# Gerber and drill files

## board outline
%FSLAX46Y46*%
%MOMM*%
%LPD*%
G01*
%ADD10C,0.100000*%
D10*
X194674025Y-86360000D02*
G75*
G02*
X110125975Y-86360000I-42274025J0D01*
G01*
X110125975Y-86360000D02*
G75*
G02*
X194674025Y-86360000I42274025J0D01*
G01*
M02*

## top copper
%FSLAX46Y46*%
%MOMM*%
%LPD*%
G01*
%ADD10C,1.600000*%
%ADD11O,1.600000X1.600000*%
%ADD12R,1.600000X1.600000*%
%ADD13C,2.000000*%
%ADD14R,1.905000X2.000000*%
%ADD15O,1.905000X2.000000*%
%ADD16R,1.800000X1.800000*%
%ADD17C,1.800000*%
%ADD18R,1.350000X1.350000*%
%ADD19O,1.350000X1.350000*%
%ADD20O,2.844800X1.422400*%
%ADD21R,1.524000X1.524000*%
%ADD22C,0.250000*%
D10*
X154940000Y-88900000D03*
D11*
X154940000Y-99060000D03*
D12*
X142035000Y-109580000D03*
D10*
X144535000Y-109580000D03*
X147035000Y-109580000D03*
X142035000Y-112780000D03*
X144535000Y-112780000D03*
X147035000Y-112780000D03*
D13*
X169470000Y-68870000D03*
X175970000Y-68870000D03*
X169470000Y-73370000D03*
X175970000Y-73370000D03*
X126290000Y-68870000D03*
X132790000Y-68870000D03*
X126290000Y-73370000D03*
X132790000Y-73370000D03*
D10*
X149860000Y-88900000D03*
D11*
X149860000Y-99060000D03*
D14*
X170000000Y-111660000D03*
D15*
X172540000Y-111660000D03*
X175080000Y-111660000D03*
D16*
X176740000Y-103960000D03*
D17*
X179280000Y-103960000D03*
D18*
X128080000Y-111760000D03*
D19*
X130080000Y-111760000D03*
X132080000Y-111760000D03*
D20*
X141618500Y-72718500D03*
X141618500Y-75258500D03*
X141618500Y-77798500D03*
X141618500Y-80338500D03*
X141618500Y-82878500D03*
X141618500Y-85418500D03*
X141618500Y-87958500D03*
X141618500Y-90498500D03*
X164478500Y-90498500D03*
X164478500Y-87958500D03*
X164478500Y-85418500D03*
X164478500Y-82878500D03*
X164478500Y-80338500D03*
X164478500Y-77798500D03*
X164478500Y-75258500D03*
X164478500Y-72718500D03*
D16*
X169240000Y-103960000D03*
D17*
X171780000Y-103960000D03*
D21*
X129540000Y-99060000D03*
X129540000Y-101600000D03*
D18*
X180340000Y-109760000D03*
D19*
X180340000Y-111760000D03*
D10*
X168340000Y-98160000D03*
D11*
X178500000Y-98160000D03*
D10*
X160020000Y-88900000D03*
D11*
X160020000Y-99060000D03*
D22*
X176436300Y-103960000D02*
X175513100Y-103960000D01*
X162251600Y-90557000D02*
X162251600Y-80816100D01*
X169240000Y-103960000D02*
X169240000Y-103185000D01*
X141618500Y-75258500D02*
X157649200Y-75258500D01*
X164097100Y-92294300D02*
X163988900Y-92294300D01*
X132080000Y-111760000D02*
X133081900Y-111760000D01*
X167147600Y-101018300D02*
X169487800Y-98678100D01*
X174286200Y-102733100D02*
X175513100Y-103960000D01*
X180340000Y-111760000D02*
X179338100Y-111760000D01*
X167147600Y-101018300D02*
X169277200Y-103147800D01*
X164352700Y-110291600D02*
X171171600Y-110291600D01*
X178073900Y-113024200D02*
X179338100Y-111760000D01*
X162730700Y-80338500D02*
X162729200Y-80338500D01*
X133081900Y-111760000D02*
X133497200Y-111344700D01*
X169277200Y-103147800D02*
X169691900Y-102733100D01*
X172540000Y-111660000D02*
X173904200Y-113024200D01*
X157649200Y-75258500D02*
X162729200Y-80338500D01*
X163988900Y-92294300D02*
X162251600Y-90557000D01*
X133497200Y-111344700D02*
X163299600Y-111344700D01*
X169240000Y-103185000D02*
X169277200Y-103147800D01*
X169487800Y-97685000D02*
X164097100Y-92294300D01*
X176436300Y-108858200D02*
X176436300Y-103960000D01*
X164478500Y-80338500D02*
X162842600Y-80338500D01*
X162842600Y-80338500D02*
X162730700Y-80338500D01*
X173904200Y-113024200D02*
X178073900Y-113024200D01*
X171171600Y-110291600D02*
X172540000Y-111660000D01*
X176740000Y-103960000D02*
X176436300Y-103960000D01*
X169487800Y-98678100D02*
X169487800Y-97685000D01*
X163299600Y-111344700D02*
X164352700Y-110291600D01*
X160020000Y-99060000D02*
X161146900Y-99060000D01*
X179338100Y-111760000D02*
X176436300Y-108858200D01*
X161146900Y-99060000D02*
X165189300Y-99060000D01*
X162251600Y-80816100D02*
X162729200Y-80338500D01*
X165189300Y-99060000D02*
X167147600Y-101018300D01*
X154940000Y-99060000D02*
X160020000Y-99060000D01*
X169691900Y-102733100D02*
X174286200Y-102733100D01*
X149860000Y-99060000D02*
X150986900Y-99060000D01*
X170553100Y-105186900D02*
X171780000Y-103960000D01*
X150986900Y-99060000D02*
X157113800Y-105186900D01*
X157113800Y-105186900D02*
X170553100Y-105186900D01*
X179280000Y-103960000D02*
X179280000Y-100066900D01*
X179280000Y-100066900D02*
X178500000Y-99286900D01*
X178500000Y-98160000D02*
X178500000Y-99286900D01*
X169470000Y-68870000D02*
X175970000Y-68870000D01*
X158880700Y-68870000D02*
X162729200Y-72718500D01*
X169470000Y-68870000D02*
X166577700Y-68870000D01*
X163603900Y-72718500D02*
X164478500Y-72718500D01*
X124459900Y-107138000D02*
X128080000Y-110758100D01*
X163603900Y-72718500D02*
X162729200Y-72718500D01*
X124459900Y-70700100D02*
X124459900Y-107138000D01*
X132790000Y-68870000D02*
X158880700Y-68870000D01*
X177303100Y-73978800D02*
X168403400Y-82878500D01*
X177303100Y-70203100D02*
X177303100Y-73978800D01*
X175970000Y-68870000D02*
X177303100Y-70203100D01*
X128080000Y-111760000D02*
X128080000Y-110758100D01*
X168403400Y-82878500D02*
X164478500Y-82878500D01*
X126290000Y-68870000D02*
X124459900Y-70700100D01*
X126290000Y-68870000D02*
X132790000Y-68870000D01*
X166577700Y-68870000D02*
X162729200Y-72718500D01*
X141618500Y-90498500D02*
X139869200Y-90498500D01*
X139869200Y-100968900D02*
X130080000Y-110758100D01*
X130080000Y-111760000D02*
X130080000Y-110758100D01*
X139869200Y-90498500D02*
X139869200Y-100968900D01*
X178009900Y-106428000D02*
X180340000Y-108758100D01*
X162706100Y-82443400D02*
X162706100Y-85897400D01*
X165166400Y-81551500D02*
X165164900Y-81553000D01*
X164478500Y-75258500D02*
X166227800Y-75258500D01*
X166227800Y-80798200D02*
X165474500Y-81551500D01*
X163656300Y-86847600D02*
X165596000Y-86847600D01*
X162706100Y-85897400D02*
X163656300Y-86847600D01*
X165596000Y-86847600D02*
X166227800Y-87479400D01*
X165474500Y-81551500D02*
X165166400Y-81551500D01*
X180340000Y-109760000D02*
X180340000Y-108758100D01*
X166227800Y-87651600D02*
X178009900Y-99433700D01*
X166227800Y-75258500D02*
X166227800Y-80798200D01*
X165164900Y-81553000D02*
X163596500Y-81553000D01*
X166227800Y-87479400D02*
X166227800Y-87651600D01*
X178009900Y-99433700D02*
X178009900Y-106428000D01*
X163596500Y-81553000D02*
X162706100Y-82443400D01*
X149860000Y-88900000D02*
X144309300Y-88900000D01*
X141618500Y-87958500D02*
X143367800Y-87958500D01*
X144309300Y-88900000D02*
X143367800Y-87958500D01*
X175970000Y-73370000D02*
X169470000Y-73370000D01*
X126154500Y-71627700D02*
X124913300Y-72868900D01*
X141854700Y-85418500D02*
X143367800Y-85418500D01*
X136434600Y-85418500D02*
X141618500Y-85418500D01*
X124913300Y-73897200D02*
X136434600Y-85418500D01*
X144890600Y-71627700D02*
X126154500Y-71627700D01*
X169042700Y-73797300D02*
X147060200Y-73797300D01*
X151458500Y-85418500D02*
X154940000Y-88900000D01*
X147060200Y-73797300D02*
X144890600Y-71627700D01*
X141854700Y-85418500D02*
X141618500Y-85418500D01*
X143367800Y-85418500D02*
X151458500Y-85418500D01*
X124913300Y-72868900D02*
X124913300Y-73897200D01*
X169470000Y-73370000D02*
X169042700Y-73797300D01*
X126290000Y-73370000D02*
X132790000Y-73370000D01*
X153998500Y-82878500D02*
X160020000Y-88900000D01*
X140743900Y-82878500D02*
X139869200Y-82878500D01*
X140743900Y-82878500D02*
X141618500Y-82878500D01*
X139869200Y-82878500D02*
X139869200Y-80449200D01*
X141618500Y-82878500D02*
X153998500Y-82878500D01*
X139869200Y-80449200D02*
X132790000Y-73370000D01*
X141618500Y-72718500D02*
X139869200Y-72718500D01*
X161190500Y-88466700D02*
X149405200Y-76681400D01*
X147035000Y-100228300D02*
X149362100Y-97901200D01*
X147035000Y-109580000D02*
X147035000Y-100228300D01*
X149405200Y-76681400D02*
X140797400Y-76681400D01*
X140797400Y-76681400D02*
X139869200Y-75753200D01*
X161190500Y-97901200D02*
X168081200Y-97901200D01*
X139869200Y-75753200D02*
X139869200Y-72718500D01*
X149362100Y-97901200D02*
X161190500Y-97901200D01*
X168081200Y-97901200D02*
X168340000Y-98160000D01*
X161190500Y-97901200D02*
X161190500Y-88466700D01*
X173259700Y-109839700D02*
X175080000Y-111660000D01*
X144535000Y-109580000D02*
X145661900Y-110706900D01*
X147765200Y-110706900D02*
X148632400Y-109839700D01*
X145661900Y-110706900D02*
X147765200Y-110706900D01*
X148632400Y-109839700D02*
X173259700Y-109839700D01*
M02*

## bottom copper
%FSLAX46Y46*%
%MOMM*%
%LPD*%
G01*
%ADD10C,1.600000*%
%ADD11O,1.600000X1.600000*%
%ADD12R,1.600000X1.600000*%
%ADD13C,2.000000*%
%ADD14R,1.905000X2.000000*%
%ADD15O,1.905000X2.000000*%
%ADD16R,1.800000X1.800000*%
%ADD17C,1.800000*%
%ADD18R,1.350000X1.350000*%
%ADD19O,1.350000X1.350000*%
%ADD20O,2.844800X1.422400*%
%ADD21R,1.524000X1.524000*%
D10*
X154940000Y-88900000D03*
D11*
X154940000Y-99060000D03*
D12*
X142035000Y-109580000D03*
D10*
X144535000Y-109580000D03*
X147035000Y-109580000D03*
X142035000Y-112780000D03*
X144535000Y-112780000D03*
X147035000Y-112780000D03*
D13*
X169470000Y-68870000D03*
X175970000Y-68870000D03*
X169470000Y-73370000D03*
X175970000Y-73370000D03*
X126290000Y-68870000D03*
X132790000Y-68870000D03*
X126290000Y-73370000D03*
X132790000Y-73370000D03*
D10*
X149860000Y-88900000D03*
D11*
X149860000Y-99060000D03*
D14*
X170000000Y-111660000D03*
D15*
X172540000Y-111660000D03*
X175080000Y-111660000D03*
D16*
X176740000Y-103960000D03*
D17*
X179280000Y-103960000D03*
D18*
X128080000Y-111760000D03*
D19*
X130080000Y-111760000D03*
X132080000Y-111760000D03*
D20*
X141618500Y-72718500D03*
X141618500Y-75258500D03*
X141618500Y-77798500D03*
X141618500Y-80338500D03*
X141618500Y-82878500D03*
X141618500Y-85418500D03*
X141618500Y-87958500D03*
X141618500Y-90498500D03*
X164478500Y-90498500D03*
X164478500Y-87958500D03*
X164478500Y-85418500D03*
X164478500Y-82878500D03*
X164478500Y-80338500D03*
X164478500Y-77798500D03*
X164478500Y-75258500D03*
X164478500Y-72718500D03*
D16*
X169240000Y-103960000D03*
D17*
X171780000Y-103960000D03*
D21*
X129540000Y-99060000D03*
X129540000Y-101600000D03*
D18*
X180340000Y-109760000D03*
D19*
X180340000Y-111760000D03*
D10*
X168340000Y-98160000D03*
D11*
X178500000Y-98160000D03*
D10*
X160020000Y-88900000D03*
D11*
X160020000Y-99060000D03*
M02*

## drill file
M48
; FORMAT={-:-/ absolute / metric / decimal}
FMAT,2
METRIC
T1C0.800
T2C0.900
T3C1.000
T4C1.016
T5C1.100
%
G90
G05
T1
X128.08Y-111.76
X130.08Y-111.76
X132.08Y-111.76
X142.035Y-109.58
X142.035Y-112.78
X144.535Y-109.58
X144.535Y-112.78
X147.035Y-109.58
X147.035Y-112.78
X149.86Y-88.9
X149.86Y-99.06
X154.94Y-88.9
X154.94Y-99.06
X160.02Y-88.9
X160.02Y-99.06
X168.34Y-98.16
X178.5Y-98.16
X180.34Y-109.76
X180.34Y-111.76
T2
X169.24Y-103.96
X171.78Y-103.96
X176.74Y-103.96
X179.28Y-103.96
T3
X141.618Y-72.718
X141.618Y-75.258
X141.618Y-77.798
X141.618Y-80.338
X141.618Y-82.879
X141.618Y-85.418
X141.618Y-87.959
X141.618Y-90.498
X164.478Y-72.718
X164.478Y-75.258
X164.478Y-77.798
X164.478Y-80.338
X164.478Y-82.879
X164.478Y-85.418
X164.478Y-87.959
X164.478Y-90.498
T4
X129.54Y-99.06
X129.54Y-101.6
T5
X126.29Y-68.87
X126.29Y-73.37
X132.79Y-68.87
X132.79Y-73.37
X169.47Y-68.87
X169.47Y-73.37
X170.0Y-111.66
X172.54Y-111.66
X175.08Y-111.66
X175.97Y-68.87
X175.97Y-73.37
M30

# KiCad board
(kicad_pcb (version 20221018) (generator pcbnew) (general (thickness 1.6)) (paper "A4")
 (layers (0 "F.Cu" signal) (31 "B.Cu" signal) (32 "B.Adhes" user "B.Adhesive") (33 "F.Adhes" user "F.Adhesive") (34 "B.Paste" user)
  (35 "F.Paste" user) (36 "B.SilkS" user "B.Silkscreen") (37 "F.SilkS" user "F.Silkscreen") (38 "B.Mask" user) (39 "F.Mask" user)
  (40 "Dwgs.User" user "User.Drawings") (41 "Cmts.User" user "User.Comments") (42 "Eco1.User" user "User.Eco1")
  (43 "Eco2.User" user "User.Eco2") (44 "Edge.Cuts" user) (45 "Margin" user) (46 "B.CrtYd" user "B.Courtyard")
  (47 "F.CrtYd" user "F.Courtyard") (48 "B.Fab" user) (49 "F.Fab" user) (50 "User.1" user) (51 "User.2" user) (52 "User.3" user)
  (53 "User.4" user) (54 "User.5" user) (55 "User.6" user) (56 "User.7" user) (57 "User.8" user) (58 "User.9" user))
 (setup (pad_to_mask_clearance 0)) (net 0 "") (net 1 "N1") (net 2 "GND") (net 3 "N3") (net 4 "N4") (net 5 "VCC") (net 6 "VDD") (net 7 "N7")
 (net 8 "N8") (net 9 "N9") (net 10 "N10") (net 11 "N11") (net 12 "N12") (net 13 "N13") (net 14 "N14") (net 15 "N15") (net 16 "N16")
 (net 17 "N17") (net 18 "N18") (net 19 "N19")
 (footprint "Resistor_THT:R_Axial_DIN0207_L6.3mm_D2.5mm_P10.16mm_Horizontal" (layer "F.Cu") (at 154.94 88.9 -90)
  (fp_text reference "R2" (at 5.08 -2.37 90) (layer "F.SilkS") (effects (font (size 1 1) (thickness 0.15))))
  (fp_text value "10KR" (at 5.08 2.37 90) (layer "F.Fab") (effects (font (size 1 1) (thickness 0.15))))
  (pad "1" thru_hole circle (at 0 0 270) (size 1.6 1.6) (drill 0.8) (layers "*.Cu" "*.Mask") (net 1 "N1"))
  (pad "2" thru_hole oval (at 10.16 0 270) (size 1.6 1.6) (drill 0.8) (layers "*.Cu" "*.Mask") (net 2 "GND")))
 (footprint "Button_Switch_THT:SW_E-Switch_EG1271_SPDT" (layer "F.Cu") (at 142.035 109.58)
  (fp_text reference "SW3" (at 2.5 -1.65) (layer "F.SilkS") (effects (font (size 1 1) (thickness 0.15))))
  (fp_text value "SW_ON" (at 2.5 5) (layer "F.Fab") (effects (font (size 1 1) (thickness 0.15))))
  (pad "1" thru_hole rect (at 0 0) (size 1.6 1.6) (drill 0.8) (layers "*.Cu" "*.Mask") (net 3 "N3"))
  (pad "2" thru_hole circle (at 2.5 0) (size 1.6 1.6) (drill 0.8) (layers "*.Cu" "*.Mask") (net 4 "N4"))
  (pad "3" thru_hole circle (at 5 0) (size 1.6 1.6) (drill 0.8) (layers "*.Cu" "*.Mask") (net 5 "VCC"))
  (pad "4" thru_hole circle (at 0 3.2) (size 1.6 1.6) (drill 0.8) (layers "*.Cu" "*.Mask"))
  (pad "5" thru_hole circle (at 2.5 3.2) (size 1.6 1.6) (drill 0.8) (layers "*.Cu" "*.Mask"))
  (pad "6" thru_hole circle (at 5 3.2) (size 1.6 1.6) (drill 0.8) (layers "*.Cu" "*.Mask")))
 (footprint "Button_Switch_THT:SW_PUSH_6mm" (layer "F.Cu") (at 169.47 68.87)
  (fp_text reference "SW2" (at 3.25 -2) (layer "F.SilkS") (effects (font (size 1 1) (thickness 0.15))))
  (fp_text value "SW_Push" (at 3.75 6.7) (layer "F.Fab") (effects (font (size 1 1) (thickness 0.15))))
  (pad "1" thru_hole circle (at 0 0 90) (size 2 2) (drill 1.1) (layers "*.Cu" "*.Mask") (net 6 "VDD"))
  (pad "1" thru_hole circle (at 6.5 0 90) (size 2 2) (drill 1.1) (layers "*.Cu" "*.Mask") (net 6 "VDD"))
  (pad "2" thru_hole circle (at 0 4.5 90) (size 2 2) (drill 1.1) (layers "*.Cu" "*.Mask") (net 1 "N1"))
  (pad "2" thru_hole circle (at 6.5 4.5 90) (size 2 2) (drill 1.1) (layers "*.Cu" "*.Mask") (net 1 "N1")))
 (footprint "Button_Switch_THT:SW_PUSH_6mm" (layer "F.Cu") (at 126.29 68.87)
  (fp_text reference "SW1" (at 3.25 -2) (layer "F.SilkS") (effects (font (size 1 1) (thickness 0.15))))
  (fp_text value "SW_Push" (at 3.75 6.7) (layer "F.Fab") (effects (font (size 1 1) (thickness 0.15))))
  (pad "1" thru_hole circle (at 0 0 90) (size 2 2) (drill 1.1) (layers "*.Cu" "*.Mask") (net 6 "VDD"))
  (pad "1" thru_hole circle (at 6.5 0 90) (size 2 2) (drill 1.1) (layers "*.Cu" "*.Mask") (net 6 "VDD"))
  (pad "2" thru_hole circle (at 0 4.5 90) (size 2 2) (drill 1.1) (layers "*.Cu" "*.Mask") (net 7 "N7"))
  (pad "2" thru_hole circle (at 6.5 4.5 90) (size 2 2) (drill 1.1) (layers "*.Cu" "*.Mask") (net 7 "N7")))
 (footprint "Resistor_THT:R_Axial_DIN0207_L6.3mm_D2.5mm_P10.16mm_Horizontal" (layer "F.Cu") (at 149.86 88.9 -90)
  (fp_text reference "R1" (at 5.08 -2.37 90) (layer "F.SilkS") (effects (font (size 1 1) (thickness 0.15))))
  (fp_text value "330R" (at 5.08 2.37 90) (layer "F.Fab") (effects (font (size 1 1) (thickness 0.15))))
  (pad "1" thru_hole circle (at 0 0 270) (size 1.6 1.6) (drill 0.8) (layers "*.Cu" "*.Mask") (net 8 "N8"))
  (pad "2" thru_hole oval (at 10.16 0 270) (size 1.6 1.6) (drill 0.8) (layers "*.Cu" "*.Mask") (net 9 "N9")))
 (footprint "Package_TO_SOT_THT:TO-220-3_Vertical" (layer "F.Cu") (at 170 111.66)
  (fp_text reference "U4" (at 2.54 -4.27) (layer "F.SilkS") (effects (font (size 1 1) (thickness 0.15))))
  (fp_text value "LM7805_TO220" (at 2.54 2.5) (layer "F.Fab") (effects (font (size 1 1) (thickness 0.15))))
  (pad "1" thru_hole rect (at 0 0) (size 1.905 2) (drill 1.1) (layers "*.Cu" "*.Mask") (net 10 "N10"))
  (pad "2" thru_hole oval (at 2.54 0) (size 1.905 2) (drill 1.1) (layers "*.Cu" "*.Mask") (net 2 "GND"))
  (pad "3" thru_hole oval (at 5.08 0) (size 1.905 2) (drill 1.1) (layers "*.Cu" "*.Mask") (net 4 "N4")))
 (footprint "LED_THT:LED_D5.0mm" (layer "F.Cu") (at 176.74 103.96)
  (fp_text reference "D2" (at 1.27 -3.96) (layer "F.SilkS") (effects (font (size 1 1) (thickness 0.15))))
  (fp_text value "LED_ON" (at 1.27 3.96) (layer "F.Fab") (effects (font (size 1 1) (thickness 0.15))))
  (pad "1" thru_hole rect (at 0 0) (size 1.8 1.8) (drill 0.9) (layers "*.Cu" "*.Mask") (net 2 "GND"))
  (pad "2" thru_hole circle (at 2.54 0) (size 1.8 1.8) (drill 0.9) (layers "*.Cu" "*.Mask") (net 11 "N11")))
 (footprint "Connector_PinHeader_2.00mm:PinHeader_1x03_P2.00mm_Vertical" (layer "F.Cu") (at 128.08 111.76 90)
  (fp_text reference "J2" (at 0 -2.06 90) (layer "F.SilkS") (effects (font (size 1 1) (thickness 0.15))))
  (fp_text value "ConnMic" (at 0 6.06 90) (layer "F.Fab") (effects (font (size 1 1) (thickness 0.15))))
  (pad "1" thru_hole rect (at 0 0 90) (size 1.35 1.35) (drill 0.8) (layers "*.Cu" "*.Mask") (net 6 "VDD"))
  (pad "2" thru_hole oval (at 0 2 90) (size 1.35 1.35) (drill 0.8) (layers "*.Cu" "*.Mask") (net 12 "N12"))
  (pad "3" thru_hole oval (at 0 4 90) (size 1.35 1.35) (drill 0.8) (layers "*.Cu" "*.Mask") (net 2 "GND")))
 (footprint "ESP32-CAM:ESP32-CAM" (layer "F.Cu") (at 153.0485 82.8785)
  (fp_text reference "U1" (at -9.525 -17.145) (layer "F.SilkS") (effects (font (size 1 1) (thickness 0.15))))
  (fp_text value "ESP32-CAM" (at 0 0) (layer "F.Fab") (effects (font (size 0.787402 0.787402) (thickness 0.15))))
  (pad "P$1" thru_hole oval (at -11.43 -10.16) (size 2.8448 1.4224) (drill 1) (layers "*.Cu" "*.Mask") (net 5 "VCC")
   (solder_mask_margin 0.102))
  (pad "P$2" thru_hole oval (at -11.43 -7.62) (size 2.8448 1.4224) (drill 1) (layers "*.Cu" "*.Mask") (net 2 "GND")
   (solder_mask_margin 0.102))
  (pad "P$3" thru_hole oval (at -11.43 -5.08) (size 2.8448 1.4224) (drill 1) (layers "*.Cu" "*.Mask") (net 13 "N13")
   (solder_mask_margin 0.102))
  (pad "P$4" thru_hole oval (at -11.43 -2.54) (size 2.8448 1.4224) (drill 1) (layers "*.Cu" "*.Mask") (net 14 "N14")
   (solder_mask_margin 0.102))
  (pad "P$5" thru_hole oval (at -11.43 0) (size 2.8448 1.4224) (drill 1) (layers "*.Cu" "*.Mask") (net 7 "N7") (solder_mask_margin 0.102))
  (pad "P$6" thru_hole oval (at -11.43 2.54) (size 2.8448 1.4224) (drill 1) (layers "*.Cu" "*.Mask") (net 1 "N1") (solder_mask_margin 0.102))
  (pad "P$7" thru_hole oval (at -11.43 5.08) (size 2.8448 1.4224) (drill 1) (layers "*.Cu" "*.Mask") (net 8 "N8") (solder_mask_margin 0.102))
  (pad "P$8" thru_hole oval (at -11.43 7.62) (size 2.8448 1.4224) (drill 1) (layers "*.Cu" "*.Mask") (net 12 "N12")
   (solder_mask_margin 0.102))
  (pad "P$9" thru_hole oval (at 11.43 7.62) (size 2.8448 1.4224) (drill 1) (layers "*.Cu" "*.Mask") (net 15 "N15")
   (solder_mask_margin 0.102))
  (pad "P$10" thru_hole oval (at 11.43 5.08) (size 2.8448 1.4224) (drill 1) (layers "*.Cu" "*.Mask") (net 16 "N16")
   (solder_mask_margin 0.102))
  (pad "P$11" thru_hole oval (at 11.43 2.54) (size 2.8448 1.4224) (drill 1) (layers "*.Cu" "*.Mask") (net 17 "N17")
   (solder_mask_margin 0.102))
  (pad "P$12" thru_hole oval (at 11.43 0) (size 2.8448 1.4224) (drill 1) (layers "*.Cu" "*.Mask") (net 6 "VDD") (solder_mask_margin 0.102))
  (pad "P$13" thru_hole oval (at 11.43 -2.54) (size 2.8448 1.4224) (drill 1) (layers "*.Cu" "*.Mask") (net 2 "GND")
   (solder_mask_margin 0.102))
  (pad "P$14" thru_hole oval (at 11.43 -5.08) (size 2.8448 1.4224) (drill 1) (layers "*.Cu" "*.Mask") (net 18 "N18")
   (solder_mask_margin 0.102))
  (pad "P$15" thru_hole oval (at 11.43 -7.62) (size 2.8448 1.4224) (drill 1) (layers "*.Cu" "*.Mask") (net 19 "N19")
   (solder_mask_margin 0.102))
  (pad "P$16" thru_hole oval (at 11.43 -10.16) (size 2.8448 1.4224) (drill 1) (layers "*.Cu" "*.Mask") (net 6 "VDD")
   (solder_mask_margin 0.102)))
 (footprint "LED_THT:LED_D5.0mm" (layer "F.Cu") (at 169.24 103.96)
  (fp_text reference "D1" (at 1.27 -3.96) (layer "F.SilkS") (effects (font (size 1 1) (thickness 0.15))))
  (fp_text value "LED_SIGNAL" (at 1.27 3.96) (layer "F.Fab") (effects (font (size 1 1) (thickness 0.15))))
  (pad "1" thru_hole rect (at 0 0) (size 1.8 1.8) (drill 0.9) (layers "*.Cu" "*.Mask") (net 2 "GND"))
  (pad "2" thru_hole circle (at 2.54 0) (size 1.8 1.8) (drill 0.9) (layers "*.Cu" "*.Mask") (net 9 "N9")))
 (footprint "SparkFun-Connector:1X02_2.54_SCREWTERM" (layer "F.Cu") (at 129.54 101.6 90)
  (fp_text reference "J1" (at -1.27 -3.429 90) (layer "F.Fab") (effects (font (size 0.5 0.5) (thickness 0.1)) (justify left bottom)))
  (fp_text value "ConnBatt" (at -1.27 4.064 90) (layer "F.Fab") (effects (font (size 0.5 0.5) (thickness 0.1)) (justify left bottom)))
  (pad "P1" thru_hole rect (at 2.54 0 90) (size 1.524 1.524) (drill 1.016) (layers "*.Cu" "*.Mask") (solder_mask_margin 0.1016)
   (thermal_bridge_angle 45))
  (pad "P2" thru_hole rect (at 0 0 90) (size 1.524 1.524) (drill 1.016) (layers "*.Cu" "*.Mask") (solder_mask_margin 0.1016)
   (thermal_bridge_angle 45)))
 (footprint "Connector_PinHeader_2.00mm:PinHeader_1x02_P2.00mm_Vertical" (layer "F.Cu") (at 180.34 109.76)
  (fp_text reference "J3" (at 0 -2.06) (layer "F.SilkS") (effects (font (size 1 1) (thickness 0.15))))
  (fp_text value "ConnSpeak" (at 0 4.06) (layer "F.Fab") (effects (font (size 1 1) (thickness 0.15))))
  (pad "1" thru_hole rect (at 0 0) (size 1.35 1.35) (drill 0.8) (layers "*.Cu" "*.Mask") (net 19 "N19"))
  (pad "2" thru_hole oval (at 0 2) (size 1.35 1.35) (drill 0.8) (layers "*.Cu" "*.Mask") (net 2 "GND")))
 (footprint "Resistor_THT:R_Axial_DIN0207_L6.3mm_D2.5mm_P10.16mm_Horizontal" (layer "F.Cu") (at 168.34 98.16)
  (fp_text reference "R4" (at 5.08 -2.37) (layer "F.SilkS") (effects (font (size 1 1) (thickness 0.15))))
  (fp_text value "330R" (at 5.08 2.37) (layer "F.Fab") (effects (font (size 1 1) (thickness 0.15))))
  (pad "1" thru_hole circle (at 0 0) (size 1.6 1.6) (drill 0.8) (layers "*.Cu" "*.Mask") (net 5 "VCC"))
  (pad "2" thru_hole oval (at 10.16 0) (size 1.6 1.6) (drill 0.8) (layers "*.Cu" "*.Mask") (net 11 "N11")))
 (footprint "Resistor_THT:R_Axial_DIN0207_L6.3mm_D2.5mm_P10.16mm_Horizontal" (layer "F.Cu") (at 160.02 88.9 -90)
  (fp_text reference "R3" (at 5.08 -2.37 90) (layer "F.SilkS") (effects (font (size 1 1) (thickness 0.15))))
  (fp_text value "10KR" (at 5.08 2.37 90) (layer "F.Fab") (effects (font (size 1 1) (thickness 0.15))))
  (pad "1" thru_hole circle (at 0 0 270) (size 1.6 1.6) (drill 0.8) (layers "*.Cu" "*.Mask") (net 7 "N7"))
  (pad "2" thru_hole oval (at 10.16 0 270) (size 1.6 1.6) (drill 0.8) (layers "*.Cu" "*.Mask") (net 2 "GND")))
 (gr_circle (center 152.4 86.36) (end 187.96 63.5) (stroke (width 0.1) (type default)) (fill none) (layer "Edge.Cuts"))
 (segment (start 176.4363 103.96) (end 175.5131 103.96) (width 0.25) (layer "F.Cu") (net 2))
 (segment (start 162.2516 90.557) (end 162.2516 80.8161) (width 0.25) (layer "F.Cu") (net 2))
 (segment (start 169.24 103.96) (end 169.24 103.185) (width 0.25) (layer "F.Cu") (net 2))
 (segment (start 141.6185 75.2585) (end 157.6492 75.2585) (width 0.25) (layer "F.Cu") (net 2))
 (segment (start 164.0971 92.2943) (end 163.9889 92.2943) (width 0.25) (layer "F.Cu") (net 2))
 (segment (start 132.08 111.76) (end 133.0819 111.76) (width 0.25) (layer "F.Cu") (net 2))
 (segment (start 167.1476 101.0183) (end 169.4878 98.6781) (width 0.25) (layer "F.Cu") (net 2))
 (segment (start 174.2862 102.7331) (end 175.5131 103.96) (width 0.25) (layer "F.Cu") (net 2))
 (segment (start 180.34 111.76) (end 179.3381 111.76) (width 0.25) (layer "F.Cu") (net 2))
 (segment (start 167.1476 101.0183) (end 169.2772 103.1478) (width 0.25) (layer "F.Cu") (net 2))
 (segment (start 164.3527 110.2916) (end 171.1716 110.2916) (width 0.25) (layer "F.Cu") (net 2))
 (segment (start 178.0739 113.0242) (end 179.3381 111.76) (width 0.25) (layer "F.Cu") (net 2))
 (segment (start 162.7307 80.3385) (end 162.7292 80.3385) (width 0.25) (layer "F.Cu") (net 2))
 (segment (start 133.0819 111.76) (end 133.4972 111.3447) (width 0.25) (layer "F.Cu") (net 2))
 (segment (start 169.2772 103.1478) (end 169.6919 102.7331) (width 0.25) (layer "F.Cu") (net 2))
 (segment (start 172.54 111.66) (end 173.9042 113.0242) (width 0.25) (layer "F.Cu") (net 2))
 (segment (start 157.6492 75.2585) (end 162.7292 80.3385) (width 0.25) (layer "F.Cu") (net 2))
 (segment (start 163.9889 92.2943) (end 162.2516 90.557) (width 0.25) (layer "F.Cu") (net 2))
 (segment (start 133.4972 111.3447) (end 163.2996 111.3447) (width 0.25) (layer "F.Cu") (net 2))
 (segment (start 169.24 103.185) (end 169.2772 103.1478) (width 0.25) (layer "F.Cu") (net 2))
 (segment (start 169.4878 97.685) (end 164.0971 92.2943) (width 0.25) (layer "F.Cu") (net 2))
 (segment (start 176.4363 108.8582) (end 176.4363 103.96) (width 0.25) (layer "F.Cu") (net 2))
 (segment (start 164.4785 80.3385) (end 162.8426 80.3385) (width 0.25) (layer "F.Cu") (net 2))
 (segment (start 162.8426 80.3385) (end 162.7307 80.3385) (width 0.25) (layer "F.Cu") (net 2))
 (segment (start 173.9042 113.0242) (end 178.0739 113.0242) (width 0.25) (layer "F.Cu") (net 2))
 (segment (start 171.1716 110.2916) (end 172.54 111.66) (width 0.25) (layer "F.Cu") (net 2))
 (segment (start 176.74 103.96) (end 176.4363 103.96) (width 0.25) (layer "F.Cu") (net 2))
 (segment (start 169.4878 98.6781) (end 169.4878 97.685) (width 0.25) (layer "F.Cu") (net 2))
 (segment (start 163.2996 111.3447) (end 164.3527 110.2916) (width 0.25) (layer "F.Cu") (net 2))
 (segment (start 160.02 99.06) (end 161.1469 99.06) (width 0.25) (layer "F.Cu") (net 2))
 (segment (start 179.3381 111.76) (end 176.4363 108.8582) (width 0.25) (layer "F.Cu") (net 2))
 (segment (start 161.1469 99.06) (end 165.1893 99.06) (width 0.25) (layer "F.Cu") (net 2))
 (segment (start 162.2516 80.8161) (end 162.7292 80.3385) (width 0.25) (layer "F.Cu") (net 2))
 (segment (start 165.1893 99.06) (end 167.1476 101.0183) (width 0.25) (layer "F.Cu") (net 2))
 (segment (start 154.94 99.06) (end 160.02 99.06) (width 0.25) (layer "F.Cu") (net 2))
 (segment (start 169.6919 102.7331) (end 174.2862 102.7331) (width 0.25) (layer "F.Cu") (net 2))
 (segment (start 149.86 99.06) (end 150.9869 99.06) (width 0.25) (layer "F.Cu") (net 9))
 (segment (start 170.5531 105.1869) (end 171.78 103.96) (width 0.25) (layer "F.Cu") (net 9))
 (segment (start 150.9869 99.06) (end 157.1138 105.1869) (width 0.25) (layer "F.Cu") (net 9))
 (segment (start 157.1138 105.1869) (end 170.5531 105.1869) (width 0.25) (layer "F.Cu") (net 9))
 (segment (start 179.28 103.96) (end 179.28 100.0669) (width 0.25) (layer "F.Cu") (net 11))
 (segment (start 179.28 100.0669) (end 178.5 99.2869) (width 0.25) (layer "F.Cu") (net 11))
 (segment (start 178.5 98.16) (end 178.5 99.2869) (width 0.25) (layer "F.Cu") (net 11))
 (segment (start 169.47 68.87) (end 175.97 68.87) (width 0.25) (layer "F.Cu") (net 6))
 (segment (start 158.8807 68.87) (end 162.7292 72.7185) (width 0.25) (layer "F.Cu") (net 6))
 (segment (start 169.47 68.87) (end 166.5777 68.87) (width 0.25) (layer "F.Cu") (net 6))
 (segment (start 163.6039 72.7185) (end 164.4785 72.7185) (width 0.25) (layer "F.Cu") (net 6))
 (segment (start 124.4599 107.138) (end 128.08 110.7581) (width 0.25) (layer "F.Cu") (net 6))
 (segment (start 163.6039 72.7185) (end 162.7292 72.7185) (width 0.25) (layer "F.Cu") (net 6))
 (segment (start 124.4599 70.7001) (end 124.4599 107.138) (width 0.25) (layer "F.Cu") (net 6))
 (segment (start 132.79 68.87) (end 158.8807 68.87) (width 0.25) (layer "F.Cu") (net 6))
 (segment (start 177.3031 73.9788) (end 168.4034 82.8785) (width 0.25) (layer "F.Cu") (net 6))
 (segment (start 177.3031 70.2031) (end 177.3031 73.9788) (width 0.25) (layer "F.Cu") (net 6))
 (segment (start 175.97 68.87) (end 177.3031 70.2031) (width 0.25) (layer "F.Cu") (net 6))
 (segment (start 128.08 111.76) (end 128.08 110.7581) (width 0.25) (layer "F.Cu") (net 6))
 (segment (start 168.4034 82.8785) (end 164.4785 82.8785) (width 0.25) (layer "F.Cu") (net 6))
 (segment (start 126.29 68.87) (end 124.4599 70.7001) (width 0.25) (layer "F.Cu") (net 6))
 (segment (start 126.29 68.87) (end 132.79 68.87) (width 0.25) (layer "F.Cu") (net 6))
 (segment (start 166.5777 68.87) (end 162.7292 72.7185) (width 0.25) (layer "F.Cu") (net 6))
 (segment (start 141.6185 90.4985) (end 139.8692 90.4985) (width 0.25) (layer "F.Cu") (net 12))
 (segment (start 139.8692 100.9689) (end 130.08 110.7581) (width 0.25) (layer "F.Cu") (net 12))
 (segment (start 130.08 111.76) (end 130.08 110.7581) (width 0.25) (layer "F.Cu") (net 12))
 (segment (start 139.8692 90.4985) (end 139.8692 100.9689) (width 0.25) (layer "F.Cu") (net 12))
 (segment (start 178.0099 106.428) (end 180.34 108.7581) (width 0.25) (layer "F.Cu") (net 19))
 (segment (start 162.7061 82.4434) (end 162.7061 85.8974) (width 0.25) (layer "F.Cu") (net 19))
 (segment (start 165.1664 81.5515) (end 165.1649 81.553) (width 0.25) (layer "F.Cu") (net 19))
 (segment (start 164.4785 75.2585) (end 166.2278 75.2585) (width 0.25) (layer "F.Cu") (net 19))
 (segment (start 166.2278 80.7982) (end 165.4745 81.5515) (width 0.25) (layer "F.Cu") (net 19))
 (segment (start 163.6563 86.8476) (end 165.596 86.8476) (width 0.25) (layer "F.Cu") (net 19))
 (segment (start 162.7061 85.8974) (end 163.6563 86.8476) (width 0.25) (layer "F.Cu") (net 19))
 (segment (start 165.596 86.8476) (end 166.2278 87.4794) (width 0.25) (layer "F.Cu") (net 19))
 (segment (start 165.4745 81.5515) (end 165.1664 81.5515) (width 0.25) (layer "F.Cu") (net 19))
 (segment (start 180.34 109.76) (end 180.34 108.7581) (width 0.25) (layer "F.Cu") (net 19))
 (segment (start 166.2278 87.6516) (end 178.0099 99.4337) (width 0.25) (layer "F.Cu") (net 19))
 (segment (start 166.2278 75.2585) (end 166.2278 80.7982) (width 0.25) (layer "F.Cu") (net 19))
 (segment (start 165.1649 81.553) (end 163.5965 81.553) (width 0.25) (layer "F.Cu") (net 19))
 (segment (start 166.2278 87.4794) (end 166.2278 87.6516) (width 0.25) (layer "F.Cu") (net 19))
 (segment (start 178.0099 99.4337) (end 178.0099 106.428) (width 0.25) (layer "F.Cu") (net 19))
 (segment (start 163.5965 81.553) (end 162.7061 82.4434) (width 0.25) (layer "F.Cu") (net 19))
 (segment (start 149.86 88.9) (end 144.3093 88.9) (width 0.25) (layer "F.Cu") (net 8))
 (segment (start 141.6185 87.9585) (end 143.3678 87.9585) (width 0.25) (layer "F.Cu") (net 8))
 (segment (start 144.3093 88.9) (end 143.3678 87.9585) (width 0.25) (layer "F.Cu") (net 8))
 (segment (start 175.97 73.37) (end 169.47 73.37) (width 0.25) (layer "F.Cu") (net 1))
 (segment (start 126.1545 71.6277) (end 124.9133 72.8689) (width 0.25) (layer "F.Cu") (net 1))
 (segment (start 141.8547 85.4185) (end 143.3678 85.4185) (width 0.25) (layer "F.Cu") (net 1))
 (segment (start 136.4346 85.4185) (end 141.6185 85.4185) (width 0.25) (layer "F.Cu") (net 1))
 (segment (start 124.9133 73.8972) (end 136.4346 85.4185) (width 0.25) (layer "F.Cu") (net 1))
 (segment (start 144.8906 71.6277) (end 126.1545 71.6277) (width 0.25) (layer "F.Cu") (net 1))
 (segment (start 169.0427 73.7973) (end 147.0602 73.7973) (width 0.25) (layer "F.Cu") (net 1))
 (segment (start 151.4585 85.4185) (end 154.94 88.9) (width 0.25) (layer "F.Cu") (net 1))
 (segment (start 147.0602 73.7973) (end 144.8906 71.6277) (width 0.25) (layer "F.Cu") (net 1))
 (segment (start 141.8547 85.4185) (end 141.6185 85.4185) (width 0.25) (layer "F.Cu") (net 1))
 (segment (start 143.3678 85.4185) (end 151.4585 85.4185) (width 0.25) (layer "F.Cu") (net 1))
 (segment (start 124.9133 72.8689) (end 124.9133 73.8972) (width 0.25) (layer "F.Cu") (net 1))
 (segment (start 169.47 73.37) (end 169.0427 73.7973) (width 0.25) (layer "F.Cu") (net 1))
 (segment (start 126.29 73.37) (end 132.79 73.37) (width 0.25) (layer "F.Cu") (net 7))
 (segment (start 153.9985 82.8785) (end 160.02 88.9) (width 0.25) (layer "F.Cu") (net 7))
 (segment (start 140.7439 82.8785) (end 139.8692 82.8785) (width 0.25) (layer "F.Cu") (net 7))
 (segment (start 140.7439 82.8785) (end 141.6185 82.8785) (width 0.25) (layer "F.Cu") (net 7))
 (segment (start 139.8692 82.8785) (end 139.8692 80.4492) (width 0.25) (layer "F.Cu") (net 7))
 (segment (start 141.6185 82.8785) (end 153.9985 82.8785) (width 0.25) (layer "F.Cu") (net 7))
 (segment (start 139.8692 80.4492) (end 132.79 73.37) (width 0.25) (layer "F.Cu") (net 7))
 (segment (start 141.6185 72.7185) (end 139.8692 72.7185) (width 0.25) (layer "F.Cu") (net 5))
 (segment (start 161.1905 88.4667) (end 149.4052 76.6814) (width 0.25) (layer "F.Cu") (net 5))
 (segment (start 147.035 100.2283) (end 149.3621 97.9012) (width 0.25) (layer "F.Cu") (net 5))
 (segment (start 147.035 109.58) (end 147.035 100.2283) (width 0.25) (layer "F.Cu") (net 5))
 (segment (start 149.4052 76.6814) (end 140.7974 76.6814) (width 0.25) (layer "F.Cu") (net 5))
 (segment (start 140.7974 76.6814) (end 139.8692 75.7532) (width 0.25) (layer "F.Cu") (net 5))
 (segment (start 161.1905 97.9012) (end 168.0812 97.9012) (width 0.25) (layer "F.Cu") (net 5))
 (segment (start 139.8692 75.7532) (end 139.8692 72.7185) (width 0.25) (layer "F.Cu") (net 5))
 (segment (start 149.3621 97.9012) (end 161.1905 97.9012) (width 0.25) (layer "F.Cu") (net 5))
 (segment (start 168.0812 97.9012) (end 168.34 98.16) (width 0.25) (layer "F.Cu") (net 5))
 (segment (start 161.1905 97.9012) (end 161.1905 88.4667) (width 0.25) (layer "F.Cu") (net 5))
 (segment (start 173.2597 109.8397) (end 175.08 111.66) (width 0.25) (layer "F.Cu") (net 4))
 (segment (start 144.535 109.58) (end 145.6619 110.7069) (width 0.25) (layer "F.Cu") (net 4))
 (segment (start 147.7652 110.7069) (end 148.6324 109.8397) (width 0.25) (layer "F.Cu") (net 4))
 (segment (start 145.6619 110.7069) (end 147.7652 110.7069) (width 0.25) (layer "F.Cu") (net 4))
 (segment (start 148.6324 109.8397) (end 173.2597 109.8397) (width 0.25) (layer "F.Cu") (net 4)))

